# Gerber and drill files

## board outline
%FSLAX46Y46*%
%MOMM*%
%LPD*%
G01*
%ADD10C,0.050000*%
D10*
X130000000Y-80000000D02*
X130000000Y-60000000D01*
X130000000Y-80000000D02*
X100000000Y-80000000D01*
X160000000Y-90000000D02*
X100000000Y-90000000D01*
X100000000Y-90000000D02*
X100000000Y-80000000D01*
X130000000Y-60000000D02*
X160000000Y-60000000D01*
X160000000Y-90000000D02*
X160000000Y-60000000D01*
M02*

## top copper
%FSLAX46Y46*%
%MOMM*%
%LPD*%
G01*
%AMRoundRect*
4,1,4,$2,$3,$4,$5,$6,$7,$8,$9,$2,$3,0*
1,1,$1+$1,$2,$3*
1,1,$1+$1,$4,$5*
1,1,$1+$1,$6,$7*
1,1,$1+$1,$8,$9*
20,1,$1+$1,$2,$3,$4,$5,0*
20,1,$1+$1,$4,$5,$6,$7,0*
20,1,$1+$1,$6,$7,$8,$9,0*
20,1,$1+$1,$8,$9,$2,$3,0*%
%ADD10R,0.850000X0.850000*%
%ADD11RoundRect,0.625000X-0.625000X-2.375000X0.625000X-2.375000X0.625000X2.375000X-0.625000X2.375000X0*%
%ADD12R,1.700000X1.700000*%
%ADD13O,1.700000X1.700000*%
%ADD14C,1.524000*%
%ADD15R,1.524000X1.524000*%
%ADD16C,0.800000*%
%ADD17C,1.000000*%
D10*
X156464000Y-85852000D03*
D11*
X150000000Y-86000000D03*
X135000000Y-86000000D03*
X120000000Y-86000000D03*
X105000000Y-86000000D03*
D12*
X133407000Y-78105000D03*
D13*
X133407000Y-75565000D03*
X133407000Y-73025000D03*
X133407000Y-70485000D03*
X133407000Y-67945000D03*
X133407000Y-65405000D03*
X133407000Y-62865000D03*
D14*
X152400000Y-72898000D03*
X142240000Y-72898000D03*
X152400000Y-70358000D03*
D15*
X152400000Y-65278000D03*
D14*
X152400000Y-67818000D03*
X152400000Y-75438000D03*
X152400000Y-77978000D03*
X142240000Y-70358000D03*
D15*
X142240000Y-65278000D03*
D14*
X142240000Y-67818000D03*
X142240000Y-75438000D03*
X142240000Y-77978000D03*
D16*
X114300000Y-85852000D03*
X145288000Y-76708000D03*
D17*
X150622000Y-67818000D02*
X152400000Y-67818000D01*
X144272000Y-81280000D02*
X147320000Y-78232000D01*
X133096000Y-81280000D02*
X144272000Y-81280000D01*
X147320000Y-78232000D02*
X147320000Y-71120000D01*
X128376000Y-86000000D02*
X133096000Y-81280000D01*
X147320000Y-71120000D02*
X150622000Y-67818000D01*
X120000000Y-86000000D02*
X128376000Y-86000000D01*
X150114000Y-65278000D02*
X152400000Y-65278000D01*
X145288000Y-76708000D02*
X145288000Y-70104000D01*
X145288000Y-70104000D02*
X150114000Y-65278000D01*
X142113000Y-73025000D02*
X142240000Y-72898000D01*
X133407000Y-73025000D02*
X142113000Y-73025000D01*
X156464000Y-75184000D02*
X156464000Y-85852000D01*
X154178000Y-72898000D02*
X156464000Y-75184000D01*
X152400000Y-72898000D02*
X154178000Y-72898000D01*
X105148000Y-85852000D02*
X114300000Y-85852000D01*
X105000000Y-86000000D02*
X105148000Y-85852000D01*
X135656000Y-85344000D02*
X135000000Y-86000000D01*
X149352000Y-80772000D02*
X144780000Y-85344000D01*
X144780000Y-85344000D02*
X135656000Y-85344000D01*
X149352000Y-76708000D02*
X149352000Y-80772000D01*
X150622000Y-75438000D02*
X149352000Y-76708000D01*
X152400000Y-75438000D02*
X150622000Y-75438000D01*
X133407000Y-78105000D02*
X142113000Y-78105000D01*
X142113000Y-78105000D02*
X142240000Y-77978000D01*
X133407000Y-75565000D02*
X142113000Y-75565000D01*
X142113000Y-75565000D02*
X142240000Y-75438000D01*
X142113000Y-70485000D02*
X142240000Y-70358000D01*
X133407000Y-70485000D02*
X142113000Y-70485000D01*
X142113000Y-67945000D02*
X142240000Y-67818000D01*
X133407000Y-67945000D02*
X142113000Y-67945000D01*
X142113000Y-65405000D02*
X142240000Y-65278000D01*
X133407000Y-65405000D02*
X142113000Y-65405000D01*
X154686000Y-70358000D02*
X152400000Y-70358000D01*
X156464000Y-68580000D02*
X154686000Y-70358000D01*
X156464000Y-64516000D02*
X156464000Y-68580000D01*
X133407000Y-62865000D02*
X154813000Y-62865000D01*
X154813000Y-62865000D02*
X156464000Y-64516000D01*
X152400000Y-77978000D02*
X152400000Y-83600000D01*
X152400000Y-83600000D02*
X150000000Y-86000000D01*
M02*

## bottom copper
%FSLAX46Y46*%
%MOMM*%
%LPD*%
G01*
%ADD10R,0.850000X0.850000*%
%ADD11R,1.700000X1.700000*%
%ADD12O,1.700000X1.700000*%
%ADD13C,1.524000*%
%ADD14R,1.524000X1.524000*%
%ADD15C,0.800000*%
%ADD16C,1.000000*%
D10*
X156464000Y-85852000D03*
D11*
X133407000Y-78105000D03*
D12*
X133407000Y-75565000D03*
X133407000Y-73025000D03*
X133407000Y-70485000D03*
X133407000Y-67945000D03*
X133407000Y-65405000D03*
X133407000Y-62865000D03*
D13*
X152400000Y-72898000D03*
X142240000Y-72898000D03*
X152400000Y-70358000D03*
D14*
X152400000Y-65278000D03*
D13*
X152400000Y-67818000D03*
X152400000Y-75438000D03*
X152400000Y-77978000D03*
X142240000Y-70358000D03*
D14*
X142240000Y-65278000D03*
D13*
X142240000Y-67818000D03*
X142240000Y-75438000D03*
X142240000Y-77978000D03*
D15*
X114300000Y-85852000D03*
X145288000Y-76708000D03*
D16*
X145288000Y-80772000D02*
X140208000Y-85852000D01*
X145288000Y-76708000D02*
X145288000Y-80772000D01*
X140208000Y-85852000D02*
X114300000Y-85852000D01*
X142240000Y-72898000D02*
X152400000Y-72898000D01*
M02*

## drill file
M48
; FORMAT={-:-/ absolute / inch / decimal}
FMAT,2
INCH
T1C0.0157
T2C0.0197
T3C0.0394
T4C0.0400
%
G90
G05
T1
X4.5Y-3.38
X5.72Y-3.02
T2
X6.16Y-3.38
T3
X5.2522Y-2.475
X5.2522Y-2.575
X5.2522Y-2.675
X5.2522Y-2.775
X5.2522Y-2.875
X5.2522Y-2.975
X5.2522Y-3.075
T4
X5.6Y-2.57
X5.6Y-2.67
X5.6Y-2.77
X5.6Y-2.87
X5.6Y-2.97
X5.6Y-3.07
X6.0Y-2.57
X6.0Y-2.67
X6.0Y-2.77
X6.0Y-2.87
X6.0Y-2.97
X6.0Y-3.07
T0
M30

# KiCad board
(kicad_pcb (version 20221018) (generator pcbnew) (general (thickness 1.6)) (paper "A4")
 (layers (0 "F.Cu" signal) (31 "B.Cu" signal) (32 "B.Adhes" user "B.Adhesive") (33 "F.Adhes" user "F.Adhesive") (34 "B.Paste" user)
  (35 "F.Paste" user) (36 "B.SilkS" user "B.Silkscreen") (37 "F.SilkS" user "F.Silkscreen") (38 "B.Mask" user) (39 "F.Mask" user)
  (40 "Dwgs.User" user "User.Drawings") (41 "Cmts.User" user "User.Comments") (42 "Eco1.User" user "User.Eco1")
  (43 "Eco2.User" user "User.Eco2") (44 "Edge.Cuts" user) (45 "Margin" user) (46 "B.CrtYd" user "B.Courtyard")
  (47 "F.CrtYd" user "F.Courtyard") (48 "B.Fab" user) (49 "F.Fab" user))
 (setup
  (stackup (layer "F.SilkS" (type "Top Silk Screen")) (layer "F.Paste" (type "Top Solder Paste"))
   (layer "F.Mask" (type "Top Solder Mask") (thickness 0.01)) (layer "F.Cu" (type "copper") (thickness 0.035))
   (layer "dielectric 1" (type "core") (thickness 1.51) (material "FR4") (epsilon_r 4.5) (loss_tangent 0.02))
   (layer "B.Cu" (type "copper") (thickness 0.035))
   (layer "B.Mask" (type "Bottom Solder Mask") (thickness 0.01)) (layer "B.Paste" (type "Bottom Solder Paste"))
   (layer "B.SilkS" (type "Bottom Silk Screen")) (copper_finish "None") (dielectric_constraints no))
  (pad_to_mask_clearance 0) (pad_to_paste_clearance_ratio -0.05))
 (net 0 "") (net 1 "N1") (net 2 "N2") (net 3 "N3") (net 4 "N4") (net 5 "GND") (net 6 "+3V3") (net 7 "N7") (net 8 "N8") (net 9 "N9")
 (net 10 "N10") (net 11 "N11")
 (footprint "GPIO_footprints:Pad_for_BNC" (layer "F.Cu") (at 104.648 91.291)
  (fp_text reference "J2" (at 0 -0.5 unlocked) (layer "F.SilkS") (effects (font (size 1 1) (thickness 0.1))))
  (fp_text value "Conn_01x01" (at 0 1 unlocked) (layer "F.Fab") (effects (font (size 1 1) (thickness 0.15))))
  (pad "1" smd roundrect (at 0.352 -5.291) (size 2.5 6) (layers "F.Cu" "F.Paste" "F.Mask") (roundrect_rratio 0.25) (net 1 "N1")
   (thermal_bridge_angle 45)))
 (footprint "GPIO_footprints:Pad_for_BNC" (layer "F.Cu") (at 118.364 91.44)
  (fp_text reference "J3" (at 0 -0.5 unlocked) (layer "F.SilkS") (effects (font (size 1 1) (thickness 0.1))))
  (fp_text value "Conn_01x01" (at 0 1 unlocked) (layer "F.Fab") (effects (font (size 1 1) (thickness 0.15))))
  (pad "1" smd roundrect (at 1.636 -5.44) (size 2.5 6) (layers "F.Cu" "F.Paste" "F.Mask") (roundrect_rratio 0.25) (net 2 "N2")
   (thermal_bridge_angle 45)))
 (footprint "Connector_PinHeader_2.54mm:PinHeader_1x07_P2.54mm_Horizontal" (layer "F.Cu") (at 133.407 78.105 180)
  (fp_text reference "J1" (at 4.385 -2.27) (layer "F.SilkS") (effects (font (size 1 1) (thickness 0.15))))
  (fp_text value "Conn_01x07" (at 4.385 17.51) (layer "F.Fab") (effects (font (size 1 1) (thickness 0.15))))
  (pad "1" thru_hole rect (at 0 0 180) (size 1.7 1.7) (drill 1) (layers "*.Cu" "*.Mask") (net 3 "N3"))
  (pad "2" thru_hole oval (at 0 2.54 180) (size 1.7 1.7) (drill 1) (layers "*.Cu" "*.Mask") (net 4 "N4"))
  (pad "3" thru_hole oval (at 0 5.08 180) (size 1.7 1.7) (drill 1) (layers "*.Cu" "*.Mask") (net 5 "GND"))
  (pad "4" thru_hole oval (at 0 7.62 180) (size 1.7 1.7) (drill 1) (layers "*.Cu" "*.Mask") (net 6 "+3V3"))
  (pad "5" thru_hole oval (at 0 10.16 180) (size 1.7 1.7) (drill 1) (layers "*.Cu" "*.Mask") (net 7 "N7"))
  (pad "6" thru_hole oval (at 0 12.7 180) (size 1.7 1.7) (drill 1) (layers "*.Cu" "*.Mask") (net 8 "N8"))
  (pad "7" thru_hole oval (at 0 15.24 180) (size 1.7 1.7) (drill 1) (layers "*.Cu" "*.Mask") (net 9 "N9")))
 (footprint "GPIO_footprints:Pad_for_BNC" (layer "F.Cu") (at 149.352 91.44)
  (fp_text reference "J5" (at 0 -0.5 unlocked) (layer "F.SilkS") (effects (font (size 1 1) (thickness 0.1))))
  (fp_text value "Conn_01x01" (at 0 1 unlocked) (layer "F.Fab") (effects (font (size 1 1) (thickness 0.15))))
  (pad "1" smd roundrect (at 0.648 -5.44) (size 2.5 6) (layers "F.Cu" "F.Paste" "F.Mask") (roundrect_rratio 0.25) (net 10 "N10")
   (thermal_bridge_angle 45)))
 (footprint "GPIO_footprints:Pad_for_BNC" (layer "F.Cu") (at 134.112 91.44)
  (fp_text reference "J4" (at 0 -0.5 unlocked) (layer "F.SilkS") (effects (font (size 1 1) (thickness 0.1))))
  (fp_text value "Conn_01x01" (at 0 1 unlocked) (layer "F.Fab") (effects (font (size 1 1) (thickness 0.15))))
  (pad "1" smd roundrect (at 0.888 -5.44) (size 2.5 6) (layers "F.Cu" "F.Paste" "F.Mask") (roundrect_rratio 0.25) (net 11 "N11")
   (thermal_bridge_angle 45)))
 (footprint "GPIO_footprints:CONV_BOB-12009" (layer "F.Cu") (at 147.32 71.628)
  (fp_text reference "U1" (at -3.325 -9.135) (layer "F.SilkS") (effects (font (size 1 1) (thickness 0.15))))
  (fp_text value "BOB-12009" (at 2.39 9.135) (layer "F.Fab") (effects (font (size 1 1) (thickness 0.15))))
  (pad "GND_1" thru_hole circle (at 5.08 1.27) (size 1.524 1.524) (drill 1.016) (layers "*.Cu" "*.Mask") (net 5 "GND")
   (solder_mask_margin 0.102))
  (pad "GND_2" thru_hole circle (at -5.08 1.27) (size 1.524 1.524) (drill 1.016) (layers "*.Cu" "*.Mask") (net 5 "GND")
   (solder_mask_margin 0.102))
  (pad "HV" thru_hole circle (at 5.08 -1.27) (size 1.524 1.524) (drill 1.016) (layers "*.Cu" "*.Mask") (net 9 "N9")
   (solder_mask_margin 0.102))
  (pad "HV1" thru_hole rect (at 5.08 -6.35) (size 1.524 1.524) (drill 1.016) (layers "*.Cu" "*.Mask") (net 1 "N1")
   (solder_mask_margin 0.102))
  (pad "HV2" thru_hole circle (at 5.08 -3.81) (size 1.524 1.524) (drill 1.016) (layers "*.Cu" "*.Mask") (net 2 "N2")
   (solder_mask_margin 0.102))
  (pad "HV3" thru_hole circle (at 5.08 3.81) (size 1.524 1.524) (drill 1.016) (layers "*.Cu" "*.Mask") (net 11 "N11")
   (solder_mask_margin 0.102))
  (pad "HV4" thru_hole circle (at 5.08 6.35) (size 1.524 1.524) (drill 1.016) (layers "*.Cu" "*.Mask") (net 10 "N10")
   (solder_mask_margin 0.102))
  (pad "LV" thru_hole circle (at -5.08 -1.27) (size 1.524 1.524) (drill 1.016) (layers "*.Cu" "*.Mask") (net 6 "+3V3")
   (solder_mask_margin 0.102))
  (pad "LV1" thru_hole rect (at -5.08 -6.35) (size 1.524 1.524) (drill 1.016) (layers "*.Cu" "*.Mask") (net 8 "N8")
   (solder_mask_margin 0.102))
  (pad "LV2" thru_hole circle (at -5.08 -3.81) (size 1.524 1.524) (drill 1.016) (layers "*.Cu" "*.Mask") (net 7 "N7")
   (solder_mask_margin 0.102))
  (pad "LV3" thru_hole circle (at -5.08 3.81) (size 1.524 1.524) (drill 1.016) (layers "*.Cu" "*.Mask") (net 4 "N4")
   (solder_mask_margin 0.102))
  (pad "LV4" thru_hole circle (at -5.08 6.35) (size 1.524 1.524) (drill 1.016) (layers "*.Cu" "*.Mask") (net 3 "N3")
   (solder_mask_margin 0.102)))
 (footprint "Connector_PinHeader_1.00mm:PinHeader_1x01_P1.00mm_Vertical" (layer "F.Cu") (at 156.464 85.852 180)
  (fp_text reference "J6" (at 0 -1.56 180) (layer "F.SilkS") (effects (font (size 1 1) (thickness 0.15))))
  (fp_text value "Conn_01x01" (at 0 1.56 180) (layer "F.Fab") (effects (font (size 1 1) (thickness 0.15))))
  (pad "1" thru_hole rect (at 0 0 180) (size 0.85 0.85) (drill 0.5) (layers "*.Cu" "*.Mask") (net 5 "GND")))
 (gr_line (start 160 90) (end 100 90) (stroke (width 0.05) (type solid)) (layer "Edge.Cuts"))
 (gr_line (start 100 90) (end 100 80) (stroke (width 0.05) (type solid)) (layer "Edge.Cuts"))
 (gr_line (start 130 80) (end 100 80) (stroke (width 0.05) (type solid)) (layer "Edge.Cuts"))
 (gr_line (start 130 80) (end 130 60) (stroke (width 0.05) (type solid)) (layer "Edge.Cuts"))
 (gr_line (start 130 60) (end 160 60) (stroke (width 0.05) (type solid)) (layer "Edge.Cuts"))
 (gr_line (start 160 90) (end 160 60) (stroke (width 0.05) (type solid)) (layer "Edge.Cuts"))
 (segment (start 142.113 78.105) (end 142.24 77.978) (width 1) (layer "F.Cu") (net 3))
 (segment (start 133.407 78.105) (end 142.113 78.105) (width 1) (layer "F.Cu") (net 3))
 (segment (start 133.407 75.565) (end 142.113 75.565) (width 1) (layer "F.Cu") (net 4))
 (segment (start 142.113 75.565) (end 142.24 75.438) (width 1) (layer "F.Cu") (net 4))
 (segment (start 142.113 70.485) (end 142.24 70.358) (width 1) (layer "F.Cu") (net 6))
 (segment (start 133.407 70.485) (end 142.113 70.485) (width 1) (layer "F.Cu") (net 6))
 (segment (start 142.113 73.025) (end 142.24 72.898) (width 1) (layer "F.Cu") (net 5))
 (segment (start 152.4 72.898) (end 154.178 72.898) (width 1) (layer "F.Cu") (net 5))
 (segment (start 154.178 72.898) (end 156.464 75.184) (width 1) (layer "F.Cu") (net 5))
 (segment (start 133.407 73.025) (end 142.113 73.025) (width 1) (layer "F.Cu") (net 5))
 (segment (start 156.464 75.184) (end 156.464 85.852) (width 1) (layer "F.Cu") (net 5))
 (segment (start 142.24 72.898) (end 152.4 72.898) (width 1) (layer "B.Cu") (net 5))
 (segment (start 142.113 65.405) (end 142.24 65.278) (width 1) (layer "F.Cu") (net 8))
 (segment (start 133.407 65.405) (end 142.113 65.405) (width 1) (layer "F.Cu") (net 8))
 (segment (start 154.686 70.358) (end 152.4 70.358) (width 1) (layer "F.Cu") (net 9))
 (segment (start 156.464 64.516) (end 156.464 68.58) (width 1) (layer "F.Cu") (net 9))
 (segment (start 156.464 68.58) (end 154.686 70.358) (width 1) (layer "F.Cu") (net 9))
 (segment (start 154.813 62.865) (end 156.464 64.516) (width 1) (layer "F.Cu") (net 9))
 (segment (start 133.407 62.865) (end 154.813 62.865) (width 1) (layer "F.Cu") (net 9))
 (segment (start 105 86) (end 105.148 85.852) (width 1) (layer "F.Cu") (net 1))
 (segment (start 145.288 76.708) (end 145.288 70.104) (width 1) (layer "F.Cu") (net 1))
 (segment (start 150.114 65.278) (end 152.4 65.278) (width 1) (layer "F.Cu") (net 1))
 (segment (start 145.288 70.104) (end 150.114 65.278) (width 1) (layer "F.Cu") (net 1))
 (segment (start 105.148 85.852) (end 114.3 85.852) (width 1) (layer "F.Cu") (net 1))
 (via (at 114.3 85.852) (size 0.8) (drill 0.4) (layers "F.Cu" "B.Cu") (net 1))
 (via (at 145.288 76.708) (size 0.8) (drill 0.4) (layers "F.Cu" "B.Cu") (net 1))
 (segment (start 145.288 76.708) (end 145.288 80.772) (width 1) (layer "B.Cu") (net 1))
 (segment (start 140.208 85.852) (end 114.3 85.852) (width 1) (layer "B.Cu") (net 1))
 (segment (start 145.288 80.772) (end 140.208 85.852) (width 1) (layer "B.Cu") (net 1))
 (segment (start 128.376 86) (end 133.096 81.28) (width 1) (layer "F.Cu") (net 2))
 (segment (start 147.32 71.12) (end 150.622 67.818) (width 1) (layer "F.Cu") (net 2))
 (segment (start 144.272 81.28) (end 147.32 78.232) (width 1) (layer "F.Cu") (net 2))
 (segment (start 147.32 78.232) (end 147.32 71.12) (width 1) (layer "F.Cu") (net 2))
 (segment (start 133.096 81.28) (end 144.272 81.28) (width 1) (layer "F.Cu") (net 2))
 (segment (start 150.622 67.818) (end 152.4 67.818) (width 1) (layer "F.Cu") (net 2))
 (segment (start 120 86) (end 128.376 86) (width 1) (layer "F.Cu") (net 2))
 (segment (start 144.78 85.344) (end 135.656 85.344) (width 1) (layer "F.Cu") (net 11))
 (segment (start 152.4 75.438) (end 150.622 75.438) (width 1) (layer "F.Cu") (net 11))
 (segment (start 135.656 85.344) (end 135 86) (width 1) (layer "F.Cu") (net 11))
 (segment (start 149.352 80.772) (end 144.78 85.344) (width 1) (layer "F.Cu") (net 11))
 (segment (start 149.352 76.708) (end 149.352 80.772) (width 1) (layer "F.Cu") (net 11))
 (segment (start 150.622 75.438) (end 149.352 76.708) (width 1) (layer "F.Cu") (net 11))
 (segment (start 152.4 77.978) (end 152.4 83.6) (width 1) (layer "F.Cu") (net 10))
 (segment (start 152.4 83.6) (end 150 86) (width 1) (layer "F.Cu") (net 10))
 (segment (start 133.407 67.945) (end 142.113 67.945) (width 1) (layer "F.Cu") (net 7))
 (segment (start 142.113 67.945) (end 142.24 67.818) (width 1) (layer "F.Cu") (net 7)))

